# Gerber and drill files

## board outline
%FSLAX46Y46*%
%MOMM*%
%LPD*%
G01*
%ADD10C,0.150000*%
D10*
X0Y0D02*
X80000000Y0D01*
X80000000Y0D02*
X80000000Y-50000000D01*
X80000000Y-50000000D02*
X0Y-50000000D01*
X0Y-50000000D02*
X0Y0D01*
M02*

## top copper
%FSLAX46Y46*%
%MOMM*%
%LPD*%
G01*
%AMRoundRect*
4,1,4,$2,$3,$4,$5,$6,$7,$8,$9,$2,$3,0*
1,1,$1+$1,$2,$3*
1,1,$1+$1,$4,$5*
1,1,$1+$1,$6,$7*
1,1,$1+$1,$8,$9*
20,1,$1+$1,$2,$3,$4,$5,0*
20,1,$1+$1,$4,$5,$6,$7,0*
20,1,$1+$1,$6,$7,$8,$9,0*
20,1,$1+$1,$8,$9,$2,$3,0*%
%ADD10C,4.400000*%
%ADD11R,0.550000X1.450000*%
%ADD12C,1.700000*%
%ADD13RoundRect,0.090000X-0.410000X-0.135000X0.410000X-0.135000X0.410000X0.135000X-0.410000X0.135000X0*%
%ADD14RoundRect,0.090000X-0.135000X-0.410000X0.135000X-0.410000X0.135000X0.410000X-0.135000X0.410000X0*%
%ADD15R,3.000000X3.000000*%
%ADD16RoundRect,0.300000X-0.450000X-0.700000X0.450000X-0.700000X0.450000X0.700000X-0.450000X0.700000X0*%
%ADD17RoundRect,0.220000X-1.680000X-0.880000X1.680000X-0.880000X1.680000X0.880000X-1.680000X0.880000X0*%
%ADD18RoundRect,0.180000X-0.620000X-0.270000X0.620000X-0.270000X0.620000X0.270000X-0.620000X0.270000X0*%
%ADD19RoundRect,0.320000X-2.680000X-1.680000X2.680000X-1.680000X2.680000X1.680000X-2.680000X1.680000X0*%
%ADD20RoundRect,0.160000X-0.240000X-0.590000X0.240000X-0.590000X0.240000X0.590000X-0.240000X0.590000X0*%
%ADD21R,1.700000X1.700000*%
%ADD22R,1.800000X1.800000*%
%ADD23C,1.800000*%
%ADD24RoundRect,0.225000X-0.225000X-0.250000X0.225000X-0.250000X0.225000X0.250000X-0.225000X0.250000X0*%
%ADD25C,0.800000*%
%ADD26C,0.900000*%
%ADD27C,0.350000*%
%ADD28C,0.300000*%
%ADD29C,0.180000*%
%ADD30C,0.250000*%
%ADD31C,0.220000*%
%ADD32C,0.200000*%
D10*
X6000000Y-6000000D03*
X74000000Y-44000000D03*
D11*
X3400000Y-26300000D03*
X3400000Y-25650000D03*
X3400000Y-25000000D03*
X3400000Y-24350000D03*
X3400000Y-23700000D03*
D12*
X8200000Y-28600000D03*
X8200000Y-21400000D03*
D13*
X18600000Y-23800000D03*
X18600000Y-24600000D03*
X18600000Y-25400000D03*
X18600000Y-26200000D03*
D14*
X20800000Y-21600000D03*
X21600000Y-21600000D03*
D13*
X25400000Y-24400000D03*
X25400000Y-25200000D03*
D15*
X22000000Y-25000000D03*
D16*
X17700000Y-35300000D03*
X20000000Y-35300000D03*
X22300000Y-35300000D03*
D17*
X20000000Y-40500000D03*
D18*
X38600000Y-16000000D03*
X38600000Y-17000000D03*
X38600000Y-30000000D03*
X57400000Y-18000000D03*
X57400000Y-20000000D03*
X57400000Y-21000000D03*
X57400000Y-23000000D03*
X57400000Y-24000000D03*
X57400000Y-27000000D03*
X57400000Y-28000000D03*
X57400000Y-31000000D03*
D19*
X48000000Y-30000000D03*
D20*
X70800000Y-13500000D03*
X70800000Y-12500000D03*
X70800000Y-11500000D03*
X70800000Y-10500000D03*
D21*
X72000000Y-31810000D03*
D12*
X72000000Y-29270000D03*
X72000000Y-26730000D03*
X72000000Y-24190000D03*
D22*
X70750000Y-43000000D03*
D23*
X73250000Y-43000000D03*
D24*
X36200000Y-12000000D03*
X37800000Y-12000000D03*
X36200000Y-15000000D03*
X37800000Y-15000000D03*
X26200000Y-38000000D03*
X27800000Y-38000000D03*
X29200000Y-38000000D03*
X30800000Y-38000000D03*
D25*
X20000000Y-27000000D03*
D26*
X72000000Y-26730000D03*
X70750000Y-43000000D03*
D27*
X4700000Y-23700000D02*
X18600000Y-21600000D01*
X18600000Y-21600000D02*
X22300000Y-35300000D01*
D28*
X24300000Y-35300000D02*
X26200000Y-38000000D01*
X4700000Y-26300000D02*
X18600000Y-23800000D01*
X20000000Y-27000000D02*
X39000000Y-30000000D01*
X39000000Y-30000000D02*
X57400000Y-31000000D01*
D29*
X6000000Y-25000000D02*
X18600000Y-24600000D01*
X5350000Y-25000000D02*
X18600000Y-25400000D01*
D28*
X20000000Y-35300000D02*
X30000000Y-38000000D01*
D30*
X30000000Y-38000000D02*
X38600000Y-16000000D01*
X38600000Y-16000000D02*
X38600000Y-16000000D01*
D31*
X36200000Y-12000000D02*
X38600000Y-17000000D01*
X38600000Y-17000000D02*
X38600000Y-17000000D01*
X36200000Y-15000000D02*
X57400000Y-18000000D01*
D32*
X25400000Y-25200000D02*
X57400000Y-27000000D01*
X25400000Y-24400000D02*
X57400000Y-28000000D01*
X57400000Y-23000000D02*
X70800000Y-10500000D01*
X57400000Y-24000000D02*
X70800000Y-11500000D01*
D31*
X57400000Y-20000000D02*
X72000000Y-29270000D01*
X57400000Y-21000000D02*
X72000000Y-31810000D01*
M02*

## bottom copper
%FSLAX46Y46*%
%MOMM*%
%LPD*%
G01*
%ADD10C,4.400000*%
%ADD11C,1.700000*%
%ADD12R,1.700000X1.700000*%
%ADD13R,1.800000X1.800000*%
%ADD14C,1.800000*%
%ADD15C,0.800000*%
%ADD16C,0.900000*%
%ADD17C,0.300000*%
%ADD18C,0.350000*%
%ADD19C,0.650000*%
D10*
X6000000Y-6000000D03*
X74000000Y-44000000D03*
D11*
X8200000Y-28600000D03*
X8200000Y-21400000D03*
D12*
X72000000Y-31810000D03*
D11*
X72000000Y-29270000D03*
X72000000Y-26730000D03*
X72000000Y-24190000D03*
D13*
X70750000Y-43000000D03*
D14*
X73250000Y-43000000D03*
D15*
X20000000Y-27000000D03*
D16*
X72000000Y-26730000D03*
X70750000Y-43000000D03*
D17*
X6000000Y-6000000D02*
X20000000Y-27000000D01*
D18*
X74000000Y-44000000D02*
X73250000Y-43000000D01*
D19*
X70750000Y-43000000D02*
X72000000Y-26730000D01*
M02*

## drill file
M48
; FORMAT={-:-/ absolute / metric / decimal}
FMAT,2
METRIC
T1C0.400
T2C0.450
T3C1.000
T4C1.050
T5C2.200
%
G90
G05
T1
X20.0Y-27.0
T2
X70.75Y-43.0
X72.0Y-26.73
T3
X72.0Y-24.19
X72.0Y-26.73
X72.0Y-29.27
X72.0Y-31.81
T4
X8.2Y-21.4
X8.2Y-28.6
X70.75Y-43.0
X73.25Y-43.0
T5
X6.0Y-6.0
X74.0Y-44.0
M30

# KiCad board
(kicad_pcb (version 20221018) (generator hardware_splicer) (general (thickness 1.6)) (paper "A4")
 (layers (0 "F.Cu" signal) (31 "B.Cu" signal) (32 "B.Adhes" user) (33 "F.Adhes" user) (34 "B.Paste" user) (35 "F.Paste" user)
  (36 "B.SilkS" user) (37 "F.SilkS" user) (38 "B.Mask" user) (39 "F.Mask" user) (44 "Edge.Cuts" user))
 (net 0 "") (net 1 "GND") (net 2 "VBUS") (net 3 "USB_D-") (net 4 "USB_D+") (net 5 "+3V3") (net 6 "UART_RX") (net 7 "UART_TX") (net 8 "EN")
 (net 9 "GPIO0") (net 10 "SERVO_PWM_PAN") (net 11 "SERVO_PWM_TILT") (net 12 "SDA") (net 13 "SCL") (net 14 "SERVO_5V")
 (gr_line (start 0 0) (end 80 0) (layer "Edge.Cuts") (width 0.15))
 (gr_line (start 80 0) (end 80 50) (layer "Edge.Cuts") (width 0.15))
 (gr_line (start 80 50) (end 0 50) (layer "Edge.Cuts") (width 0.15))
 (gr_line (start 0 50) (end 0 0) (layer "Edge.Cuts") (width 0.15))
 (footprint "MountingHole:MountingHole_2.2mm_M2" (layer "F.Cu") (at 6 6 0) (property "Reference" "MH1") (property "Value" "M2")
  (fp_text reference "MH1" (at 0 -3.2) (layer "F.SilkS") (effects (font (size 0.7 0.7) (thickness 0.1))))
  (pad "1" thru_hole circle (at 0 0) (size 4.4 4.4) (drill 2.2) (layers "*.Cu" "*.Mask") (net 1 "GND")))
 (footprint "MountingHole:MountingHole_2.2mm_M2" (layer "F.Cu") (at 74 44 0) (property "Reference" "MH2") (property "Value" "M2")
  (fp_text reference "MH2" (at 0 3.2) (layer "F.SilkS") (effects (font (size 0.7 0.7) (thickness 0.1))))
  (pad "1" thru_hole circle (at 0 0) (size 4.4 4.4) (drill 2.2) (layers "*.Cu" "*.Mask") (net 1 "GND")))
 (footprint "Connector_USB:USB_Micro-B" (layer "F.Cu") (at 6 25 90) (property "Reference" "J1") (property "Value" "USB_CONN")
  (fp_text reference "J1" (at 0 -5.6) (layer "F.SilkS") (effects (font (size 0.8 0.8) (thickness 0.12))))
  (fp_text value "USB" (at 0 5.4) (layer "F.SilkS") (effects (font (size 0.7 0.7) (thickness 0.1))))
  (pad "1" smd rect (at -1.3 -2.6) (size 0.55 1.45) (layers "F.Cu" "F.Mask" "F.Paste") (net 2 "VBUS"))
  (pad "2" smd rect (at -0.65 -2.6) (size 0.55 1.45) (layers "F.Cu" "F.Mask" "F.Paste") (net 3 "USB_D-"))
  (pad "3" smd rect (at 0 -2.6) (size 0.55 1.45) (layers "F.Cu" "F.Mask" "F.Paste") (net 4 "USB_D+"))
  (pad "4" smd rect (at 0.65 -2.6) (size 0.55 1.45) (layers "F.Cu" "F.Mask" "F.Paste") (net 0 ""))
  (pad "5" smd rect (at 1.3 -2.6) (size 0.55 1.45) (layers "F.Cu" "F.Mask" "F.Paste") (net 1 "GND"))
  (pad "MH1" thru_hole circle (at -3.6 2.2) (size 1.7 1.7) (drill 1.05) (layers "*.Cu" "*.Mask") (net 1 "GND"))
  (pad "MH2" thru_hole circle (at 3.6 2.2) (size 1.7 1.7) (drill 1.05) (layers "*.Cu" "*.Mask") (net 1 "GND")))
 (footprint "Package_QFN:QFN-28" (layer "F.Cu") (at 22 25 0) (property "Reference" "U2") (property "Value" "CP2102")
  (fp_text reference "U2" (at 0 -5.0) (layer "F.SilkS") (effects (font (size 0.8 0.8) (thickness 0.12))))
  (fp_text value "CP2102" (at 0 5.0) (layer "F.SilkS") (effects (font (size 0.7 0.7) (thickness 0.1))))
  (pad "3" smd roundrect (at -3.4 -1.2) (size 1.0 0.45) (layers "F.Cu" "F.Mask" "F.Paste") (roundrect_rratio 0.2) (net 1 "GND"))
  (pad "4" smd roundrect (at -3.4 -0.4) (size 1.0 0.45) (layers "F.Cu" "F.Mask" "F.Paste") (roundrect_rratio 0.2) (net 4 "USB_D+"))
  (pad "5" smd roundrect (at -3.4 0.4) (size 1.0 0.45) (layers "F.Cu" "F.Mask" "F.Paste") (roundrect_rratio 0.2) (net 3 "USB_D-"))
  (pad "6" smd roundrect (at -3.4 1.2) (size 1.0 0.45) (layers "F.Cu" "F.Mask" "F.Paste") (roundrect_rratio 0.2) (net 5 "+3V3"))
  (pad "7" smd roundrect (at -1.2 -3.4) (size 0.45 1.0) (layers "F.Cu" "F.Mask" "F.Paste") (roundrect_rratio 0.2) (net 2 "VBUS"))
  (pad "8" smd roundrect (at -0.4 -3.4) (size 0.45 1.0) (layers "F.Cu" "F.Mask" "F.Paste") (roundrect_rratio 0.2) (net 2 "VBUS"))
  (pad "22" smd roundrect (at 3.4 -0.6) (size 1.0 0.45) (layers "F.Cu" "F.Mask" "F.Paste") (roundrect_rratio 0.2) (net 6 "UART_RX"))
  (pad "23" smd roundrect (at 3.4 0.2) (size 1.0 0.45) (layers "F.Cu" "F.Mask" "F.Paste") (roundrect_rratio 0.2) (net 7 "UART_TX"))
  (pad "29" smd rect (at 0 0) (size 3.0 3.0) (layers "F.Cu" "F.Mask" "F.Paste") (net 1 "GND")))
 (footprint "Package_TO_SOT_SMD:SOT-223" (layer "F.Cu") (at 20 38 0) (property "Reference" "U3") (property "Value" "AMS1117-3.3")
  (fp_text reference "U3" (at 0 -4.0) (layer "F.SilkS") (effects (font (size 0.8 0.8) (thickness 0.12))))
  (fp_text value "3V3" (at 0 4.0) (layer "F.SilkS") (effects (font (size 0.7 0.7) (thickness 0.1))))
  (pad "1" smd roundrect (at -2.3 -2.7) (size 1.5 2.0) (layers "F.Cu" "F.Mask" "F.Paste") (roundrect_rratio 0.2) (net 1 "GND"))
  (pad "2" smd roundrect (at 0 -2.7) (size 1.5 2.0) (layers "F.Cu" "F.Mask" "F.Paste") (roundrect_rratio 0.2) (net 5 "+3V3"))
  (pad "3" smd roundrect (at 2.3 -2.7) (size 1.5 2.0) (layers "F.Cu" "F.Mask" "F.Paste") (roundrect_rratio 0.2) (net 2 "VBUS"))
  (pad "4" smd roundrect (at 0 2.5) (size 3.8 2.2) (layers "F.Cu" "F.Mask" "F.Paste") (roundrect_rratio 0.1) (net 5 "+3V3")))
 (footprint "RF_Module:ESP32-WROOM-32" (layer "F.Cu") (at 48 24 0) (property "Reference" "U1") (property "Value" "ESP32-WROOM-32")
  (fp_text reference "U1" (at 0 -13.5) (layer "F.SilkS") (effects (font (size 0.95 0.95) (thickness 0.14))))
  (pad "1" smd roundrect (at -9.4 -8.0) (size 1.6 0.9) (layers "F.Cu" "F.Mask" "F.Paste") (roundrect_rratio 0.2) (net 5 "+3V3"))
  (pad "2" smd roundrect (at -9.4 -7.0) (size 1.6 0.9) (layers "F.Cu" "F.Mask" "F.Paste") (roundrect_rratio 0.2) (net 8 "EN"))
  (pad "15" smd roundrect (at -9.4 6.0) (size 1.6 0.9) (layers "F.Cu" "F.Mask" "F.Paste") (roundrect_rratio 0.2) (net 1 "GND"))
  (pad "25" smd roundrect (at 9.4 -6.0) (size 1.6 0.9) (layers "F.Cu" "F.Mask" "F.Paste") (roundrect_rratio 0.2) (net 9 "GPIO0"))
  (pad "27" smd roundrect (at 9.4 -4.0) (size 1.6 0.9) (layers "F.Cu" "F.Mask" "F.Paste") (roundrect_rratio 0.2) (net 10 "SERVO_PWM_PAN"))
  (pad "28" smd roundrect (at 9.4 -3.0) (size 1.6 0.9) (layers "F.Cu" "F.Mask" "F.Paste") (roundrect_rratio 0.2) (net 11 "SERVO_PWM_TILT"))
  (pad "30" smd roundrect (at 9.4 -1.0) (size 1.6 0.9) (layers "F.Cu" "F.Mask" "F.Paste") (roundrect_rratio 0.2) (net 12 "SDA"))
  (pad "31" smd roundrect (at 9.4 0.0) (size 1.6 0.9) (layers "F.Cu" "F.Mask" "F.Paste") (roundrect_rratio 0.2) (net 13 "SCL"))
  (pad "34" smd roundrect (at 9.4 3.0) (size 1.6 0.9) (layers "F.Cu" "F.Mask" "F.Paste") (roundrect_rratio 0.2) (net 7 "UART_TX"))
  (pad "35" smd roundrect (at 9.4 4.0) (size 1.6 0.9) (layers "F.Cu" "F.Mask" "F.Paste") (roundrect_rratio 0.2) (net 6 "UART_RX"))
  (pad "38" smd roundrect (at 9.4 7.0) (size 1.6 0.9) (layers "F.Cu" "F.Mask" "F.Paste") (roundrect_rratio 0.2) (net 1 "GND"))
  (pad "EP" smd roundrect (at 0 6.0) (size 6.0 4.0) (layers "F.Cu" "F.Mask" "F.Paste") (roundrect_rratio 0.08) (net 1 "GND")))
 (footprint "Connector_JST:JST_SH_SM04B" (layer "F.Cu") (at 72 12 90) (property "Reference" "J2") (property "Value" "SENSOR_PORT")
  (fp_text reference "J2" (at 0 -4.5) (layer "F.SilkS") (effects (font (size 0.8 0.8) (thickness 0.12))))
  (pad "1" smd roundrect (at -1.5 -1.2) (size 0.8 1.5) (layers "F.Cu" "F.Mask" "F.Paste") (roundrect_rratio 0.2) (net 12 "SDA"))
  (pad "2" smd roundrect (at -0.5 -1.2) (size 0.8 1.5) (layers "F.Cu" "F.Mask" "F.Paste") (roundrect_rratio 0.2) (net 13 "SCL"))
  (pad "3" smd roundrect (at 0.5 -1.2) (size 0.8 1.5) (layers "F.Cu" "F.Mask" "F.Paste") (roundrect_rratio 0.2) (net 5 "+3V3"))
  (pad "4" smd roundrect (at 1.5 -1.2) (size 0.8 1.5) (layers "F.Cu" "F.Mask" "F.Paste") (roundrect_rratio 0.2) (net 1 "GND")))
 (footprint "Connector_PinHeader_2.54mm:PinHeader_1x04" (layer "F.Cu") (at 72 28 90) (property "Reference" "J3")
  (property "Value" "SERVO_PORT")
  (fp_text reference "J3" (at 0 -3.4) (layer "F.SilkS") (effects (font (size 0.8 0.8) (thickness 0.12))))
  (pad "1" thru_hole rect (at -3.81 0) (size 1.7 1.7) (drill 1.0) (layers "*.Cu" "*.Mask") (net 1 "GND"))
  (pad "2" thru_hole circle (at -1.27 0) (size 1.7 1.7) (drill 1.0) (layers "*.Cu" "*.Mask") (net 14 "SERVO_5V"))
  (pad "3" thru_hole circle (at 1.27 0) (size 1.7 1.7) (drill 1.0) (layers "*.Cu" "*.Mask") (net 10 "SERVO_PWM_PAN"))
  (pad "4" thru_hole circle (at 3.81 0) (size 1.7 1.7) (drill 1.0) (layers "*.Cu" "*.Mask") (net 11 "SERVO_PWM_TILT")))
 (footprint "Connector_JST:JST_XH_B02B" (layer "F.Cu") (at 72 43 0) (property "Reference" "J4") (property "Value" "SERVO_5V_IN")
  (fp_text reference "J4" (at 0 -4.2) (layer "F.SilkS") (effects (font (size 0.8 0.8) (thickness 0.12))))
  (pad "1" thru_hole rect (at -1.25 0) (size 1.8 1.8) (drill 1.05) (layers "*.Cu" "*.Mask") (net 14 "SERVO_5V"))
  (pad "2" thru_hole circle (at 1.25 0) (size 1.8 1.8) (drill 1.05) (layers "*.Cu" "*.Mask") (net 1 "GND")))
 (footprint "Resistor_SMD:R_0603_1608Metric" (layer "F.Cu") (at 37 12 0) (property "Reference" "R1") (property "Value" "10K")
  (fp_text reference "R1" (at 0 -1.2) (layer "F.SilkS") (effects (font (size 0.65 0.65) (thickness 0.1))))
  (pad "1" smd roundrect (at -0.8 0) (size 0.9 0.95) (layers "F.Cu" "F.Mask" "F.Paste") (roundrect_rratio 0.25) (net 5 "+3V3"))
  (pad "2" smd roundrect (at 0.8 0) (size 0.9 0.95) (layers "F.Cu" "F.Mask" "F.Paste") (roundrect_rratio 0.25) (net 8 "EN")))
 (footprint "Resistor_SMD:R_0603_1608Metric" (layer "F.Cu") (at 37 15 0) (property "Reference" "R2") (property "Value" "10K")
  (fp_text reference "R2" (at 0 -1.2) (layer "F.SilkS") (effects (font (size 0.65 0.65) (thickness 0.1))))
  (pad "1" smd roundrect (at -0.8 0) (size 0.9 0.95) (layers "F.Cu" "F.Mask" "F.Paste") (roundrect_rratio 0.25) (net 5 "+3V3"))
  (pad "2" smd roundrect (at 0.8 0) (size 0.9 0.95) (layers "F.Cu" "F.Mask" "F.Paste") (roundrect_rratio 0.25) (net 9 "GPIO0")))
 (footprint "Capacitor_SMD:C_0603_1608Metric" (layer "F.Cu") (at 27 38 0) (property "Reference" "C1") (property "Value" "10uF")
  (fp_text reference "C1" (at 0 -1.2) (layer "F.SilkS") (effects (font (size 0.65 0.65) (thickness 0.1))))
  (pad "1" smd roundrect (at -0.8 0) (size 0.9 0.95) (layers "F.Cu" "F.Mask" "F.Paste") (roundrect_rratio 0.25) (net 2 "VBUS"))
  (pad "2" smd roundrect (at 0.8 0) (size 0.9 0.95) (layers "F.Cu" "F.Mask" "F.Paste") (roundrect_rratio 0.25) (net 1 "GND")))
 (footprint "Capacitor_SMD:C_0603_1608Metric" (layer "F.Cu") (at 30 38 0) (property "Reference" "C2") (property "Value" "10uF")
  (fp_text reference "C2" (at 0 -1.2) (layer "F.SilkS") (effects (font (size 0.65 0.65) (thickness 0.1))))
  (pad "1" smd roundrect (at -0.8 0) (size 0.9 0.95) (layers "F.Cu" "F.Mask" "F.Paste") (roundrect_rratio 0.25) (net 5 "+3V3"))
  (pad "2" smd roundrect (at 0.8 0) (size 0.9 0.95) (layers "F.Cu" "F.Mask" "F.Paste") (roundrect_rratio 0.25) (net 1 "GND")))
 (segment (start 4.7 23.7) (end 18.6 21.6) (width 0.35) (layer "F.Cu") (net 2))
 (segment (start 18.6 21.6) (end 22.3 35.3) (width 0.35) (layer "F.Cu") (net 2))
 (segment (start 24.3 35.3) (end 26.2 38) (width 0.3) (layer "F.Cu") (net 2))
 (segment (start 4.7 26.3) (end 18.6 23.8) (width 0.3) (layer "F.Cu") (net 1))
 (segment (start 20 27) (end 39 30) (width 0.3) (layer "F.Cu") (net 1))
 (segment (start 39 30) (end 57.4 31) (width 0.3) (layer "F.Cu") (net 1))
 (segment (start 6 6) (end 20 27) (width 0.3) (layer "B.Cu") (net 1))
 (segment (start 74 44) (end 73.25 43) (width 0.35) (layer "B.Cu") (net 1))
 (segment (start 6 25) (end 18.6 24.6) (width 0.18) (layer "F.Cu") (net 4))
 (segment (start 5.35 25) (end 18.6 25.4) (width 0.18) (layer "F.Cu") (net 3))
 (segment (start 20 35.3) (end 30 38) (width 0.3) (layer "F.Cu") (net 5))
 (segment (start 30 38) (end 38.6 16) (width 0.25) (layer "F.Cu") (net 5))
 (segment (start 38.6 16) (end 38.6 16) (width 0.25) (layer "F.Cu") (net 5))
 (segment (start 36.2 12) (end 38.6 17) (width 0.22) (layer "F.Cu") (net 8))
 (segment (start 38.6 17) (end 38.6 17) (width 0.22) (layer "F.Cu") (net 8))
 (segment (start 36.2 15) (end 57.4 18) (width 0.22) (layer "F.Cu") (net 9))
 (segment (start 25.4 25.2) (end 57.4 27) (width 0.2) (layer "F.Cu") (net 7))
 (segment (start 25.4 24.4) (end 57.4 28) (width 0.2) (layer "F.Cu") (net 6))
 (segment (start 57.4 23) (end 70.8 10.5) (width 0.2) (layer "F.Cu") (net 12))
 (segment (start 57.4 24) (end 70.8 11.5) (width 0.2) (layer "F.Cu") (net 13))
 (segment (start 70.75 43) (end 72 26.73) (width 0.65) (layer "B.Cu") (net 14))
 (segment (start 57.4 20) (end 72 29.27) (width 0.22) (layer "F.Cu") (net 10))
 (segment (start 57.4 21) (end 72 31.81) (width 0.22) (layer "F.Cu") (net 11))
 (via (at 20 27) (size 0.8) (drill 0.4) (layers "F.Cu" "B.Cu") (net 1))
 (via (at 72 26.73) (size 0.9) (drill 0.45) (layers "F.Cu" "B.Cu") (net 14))
 (via (at 70.75 43) (size 0.9) (drill 0.45) (layers "F.Cu" "B.Cu") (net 14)))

